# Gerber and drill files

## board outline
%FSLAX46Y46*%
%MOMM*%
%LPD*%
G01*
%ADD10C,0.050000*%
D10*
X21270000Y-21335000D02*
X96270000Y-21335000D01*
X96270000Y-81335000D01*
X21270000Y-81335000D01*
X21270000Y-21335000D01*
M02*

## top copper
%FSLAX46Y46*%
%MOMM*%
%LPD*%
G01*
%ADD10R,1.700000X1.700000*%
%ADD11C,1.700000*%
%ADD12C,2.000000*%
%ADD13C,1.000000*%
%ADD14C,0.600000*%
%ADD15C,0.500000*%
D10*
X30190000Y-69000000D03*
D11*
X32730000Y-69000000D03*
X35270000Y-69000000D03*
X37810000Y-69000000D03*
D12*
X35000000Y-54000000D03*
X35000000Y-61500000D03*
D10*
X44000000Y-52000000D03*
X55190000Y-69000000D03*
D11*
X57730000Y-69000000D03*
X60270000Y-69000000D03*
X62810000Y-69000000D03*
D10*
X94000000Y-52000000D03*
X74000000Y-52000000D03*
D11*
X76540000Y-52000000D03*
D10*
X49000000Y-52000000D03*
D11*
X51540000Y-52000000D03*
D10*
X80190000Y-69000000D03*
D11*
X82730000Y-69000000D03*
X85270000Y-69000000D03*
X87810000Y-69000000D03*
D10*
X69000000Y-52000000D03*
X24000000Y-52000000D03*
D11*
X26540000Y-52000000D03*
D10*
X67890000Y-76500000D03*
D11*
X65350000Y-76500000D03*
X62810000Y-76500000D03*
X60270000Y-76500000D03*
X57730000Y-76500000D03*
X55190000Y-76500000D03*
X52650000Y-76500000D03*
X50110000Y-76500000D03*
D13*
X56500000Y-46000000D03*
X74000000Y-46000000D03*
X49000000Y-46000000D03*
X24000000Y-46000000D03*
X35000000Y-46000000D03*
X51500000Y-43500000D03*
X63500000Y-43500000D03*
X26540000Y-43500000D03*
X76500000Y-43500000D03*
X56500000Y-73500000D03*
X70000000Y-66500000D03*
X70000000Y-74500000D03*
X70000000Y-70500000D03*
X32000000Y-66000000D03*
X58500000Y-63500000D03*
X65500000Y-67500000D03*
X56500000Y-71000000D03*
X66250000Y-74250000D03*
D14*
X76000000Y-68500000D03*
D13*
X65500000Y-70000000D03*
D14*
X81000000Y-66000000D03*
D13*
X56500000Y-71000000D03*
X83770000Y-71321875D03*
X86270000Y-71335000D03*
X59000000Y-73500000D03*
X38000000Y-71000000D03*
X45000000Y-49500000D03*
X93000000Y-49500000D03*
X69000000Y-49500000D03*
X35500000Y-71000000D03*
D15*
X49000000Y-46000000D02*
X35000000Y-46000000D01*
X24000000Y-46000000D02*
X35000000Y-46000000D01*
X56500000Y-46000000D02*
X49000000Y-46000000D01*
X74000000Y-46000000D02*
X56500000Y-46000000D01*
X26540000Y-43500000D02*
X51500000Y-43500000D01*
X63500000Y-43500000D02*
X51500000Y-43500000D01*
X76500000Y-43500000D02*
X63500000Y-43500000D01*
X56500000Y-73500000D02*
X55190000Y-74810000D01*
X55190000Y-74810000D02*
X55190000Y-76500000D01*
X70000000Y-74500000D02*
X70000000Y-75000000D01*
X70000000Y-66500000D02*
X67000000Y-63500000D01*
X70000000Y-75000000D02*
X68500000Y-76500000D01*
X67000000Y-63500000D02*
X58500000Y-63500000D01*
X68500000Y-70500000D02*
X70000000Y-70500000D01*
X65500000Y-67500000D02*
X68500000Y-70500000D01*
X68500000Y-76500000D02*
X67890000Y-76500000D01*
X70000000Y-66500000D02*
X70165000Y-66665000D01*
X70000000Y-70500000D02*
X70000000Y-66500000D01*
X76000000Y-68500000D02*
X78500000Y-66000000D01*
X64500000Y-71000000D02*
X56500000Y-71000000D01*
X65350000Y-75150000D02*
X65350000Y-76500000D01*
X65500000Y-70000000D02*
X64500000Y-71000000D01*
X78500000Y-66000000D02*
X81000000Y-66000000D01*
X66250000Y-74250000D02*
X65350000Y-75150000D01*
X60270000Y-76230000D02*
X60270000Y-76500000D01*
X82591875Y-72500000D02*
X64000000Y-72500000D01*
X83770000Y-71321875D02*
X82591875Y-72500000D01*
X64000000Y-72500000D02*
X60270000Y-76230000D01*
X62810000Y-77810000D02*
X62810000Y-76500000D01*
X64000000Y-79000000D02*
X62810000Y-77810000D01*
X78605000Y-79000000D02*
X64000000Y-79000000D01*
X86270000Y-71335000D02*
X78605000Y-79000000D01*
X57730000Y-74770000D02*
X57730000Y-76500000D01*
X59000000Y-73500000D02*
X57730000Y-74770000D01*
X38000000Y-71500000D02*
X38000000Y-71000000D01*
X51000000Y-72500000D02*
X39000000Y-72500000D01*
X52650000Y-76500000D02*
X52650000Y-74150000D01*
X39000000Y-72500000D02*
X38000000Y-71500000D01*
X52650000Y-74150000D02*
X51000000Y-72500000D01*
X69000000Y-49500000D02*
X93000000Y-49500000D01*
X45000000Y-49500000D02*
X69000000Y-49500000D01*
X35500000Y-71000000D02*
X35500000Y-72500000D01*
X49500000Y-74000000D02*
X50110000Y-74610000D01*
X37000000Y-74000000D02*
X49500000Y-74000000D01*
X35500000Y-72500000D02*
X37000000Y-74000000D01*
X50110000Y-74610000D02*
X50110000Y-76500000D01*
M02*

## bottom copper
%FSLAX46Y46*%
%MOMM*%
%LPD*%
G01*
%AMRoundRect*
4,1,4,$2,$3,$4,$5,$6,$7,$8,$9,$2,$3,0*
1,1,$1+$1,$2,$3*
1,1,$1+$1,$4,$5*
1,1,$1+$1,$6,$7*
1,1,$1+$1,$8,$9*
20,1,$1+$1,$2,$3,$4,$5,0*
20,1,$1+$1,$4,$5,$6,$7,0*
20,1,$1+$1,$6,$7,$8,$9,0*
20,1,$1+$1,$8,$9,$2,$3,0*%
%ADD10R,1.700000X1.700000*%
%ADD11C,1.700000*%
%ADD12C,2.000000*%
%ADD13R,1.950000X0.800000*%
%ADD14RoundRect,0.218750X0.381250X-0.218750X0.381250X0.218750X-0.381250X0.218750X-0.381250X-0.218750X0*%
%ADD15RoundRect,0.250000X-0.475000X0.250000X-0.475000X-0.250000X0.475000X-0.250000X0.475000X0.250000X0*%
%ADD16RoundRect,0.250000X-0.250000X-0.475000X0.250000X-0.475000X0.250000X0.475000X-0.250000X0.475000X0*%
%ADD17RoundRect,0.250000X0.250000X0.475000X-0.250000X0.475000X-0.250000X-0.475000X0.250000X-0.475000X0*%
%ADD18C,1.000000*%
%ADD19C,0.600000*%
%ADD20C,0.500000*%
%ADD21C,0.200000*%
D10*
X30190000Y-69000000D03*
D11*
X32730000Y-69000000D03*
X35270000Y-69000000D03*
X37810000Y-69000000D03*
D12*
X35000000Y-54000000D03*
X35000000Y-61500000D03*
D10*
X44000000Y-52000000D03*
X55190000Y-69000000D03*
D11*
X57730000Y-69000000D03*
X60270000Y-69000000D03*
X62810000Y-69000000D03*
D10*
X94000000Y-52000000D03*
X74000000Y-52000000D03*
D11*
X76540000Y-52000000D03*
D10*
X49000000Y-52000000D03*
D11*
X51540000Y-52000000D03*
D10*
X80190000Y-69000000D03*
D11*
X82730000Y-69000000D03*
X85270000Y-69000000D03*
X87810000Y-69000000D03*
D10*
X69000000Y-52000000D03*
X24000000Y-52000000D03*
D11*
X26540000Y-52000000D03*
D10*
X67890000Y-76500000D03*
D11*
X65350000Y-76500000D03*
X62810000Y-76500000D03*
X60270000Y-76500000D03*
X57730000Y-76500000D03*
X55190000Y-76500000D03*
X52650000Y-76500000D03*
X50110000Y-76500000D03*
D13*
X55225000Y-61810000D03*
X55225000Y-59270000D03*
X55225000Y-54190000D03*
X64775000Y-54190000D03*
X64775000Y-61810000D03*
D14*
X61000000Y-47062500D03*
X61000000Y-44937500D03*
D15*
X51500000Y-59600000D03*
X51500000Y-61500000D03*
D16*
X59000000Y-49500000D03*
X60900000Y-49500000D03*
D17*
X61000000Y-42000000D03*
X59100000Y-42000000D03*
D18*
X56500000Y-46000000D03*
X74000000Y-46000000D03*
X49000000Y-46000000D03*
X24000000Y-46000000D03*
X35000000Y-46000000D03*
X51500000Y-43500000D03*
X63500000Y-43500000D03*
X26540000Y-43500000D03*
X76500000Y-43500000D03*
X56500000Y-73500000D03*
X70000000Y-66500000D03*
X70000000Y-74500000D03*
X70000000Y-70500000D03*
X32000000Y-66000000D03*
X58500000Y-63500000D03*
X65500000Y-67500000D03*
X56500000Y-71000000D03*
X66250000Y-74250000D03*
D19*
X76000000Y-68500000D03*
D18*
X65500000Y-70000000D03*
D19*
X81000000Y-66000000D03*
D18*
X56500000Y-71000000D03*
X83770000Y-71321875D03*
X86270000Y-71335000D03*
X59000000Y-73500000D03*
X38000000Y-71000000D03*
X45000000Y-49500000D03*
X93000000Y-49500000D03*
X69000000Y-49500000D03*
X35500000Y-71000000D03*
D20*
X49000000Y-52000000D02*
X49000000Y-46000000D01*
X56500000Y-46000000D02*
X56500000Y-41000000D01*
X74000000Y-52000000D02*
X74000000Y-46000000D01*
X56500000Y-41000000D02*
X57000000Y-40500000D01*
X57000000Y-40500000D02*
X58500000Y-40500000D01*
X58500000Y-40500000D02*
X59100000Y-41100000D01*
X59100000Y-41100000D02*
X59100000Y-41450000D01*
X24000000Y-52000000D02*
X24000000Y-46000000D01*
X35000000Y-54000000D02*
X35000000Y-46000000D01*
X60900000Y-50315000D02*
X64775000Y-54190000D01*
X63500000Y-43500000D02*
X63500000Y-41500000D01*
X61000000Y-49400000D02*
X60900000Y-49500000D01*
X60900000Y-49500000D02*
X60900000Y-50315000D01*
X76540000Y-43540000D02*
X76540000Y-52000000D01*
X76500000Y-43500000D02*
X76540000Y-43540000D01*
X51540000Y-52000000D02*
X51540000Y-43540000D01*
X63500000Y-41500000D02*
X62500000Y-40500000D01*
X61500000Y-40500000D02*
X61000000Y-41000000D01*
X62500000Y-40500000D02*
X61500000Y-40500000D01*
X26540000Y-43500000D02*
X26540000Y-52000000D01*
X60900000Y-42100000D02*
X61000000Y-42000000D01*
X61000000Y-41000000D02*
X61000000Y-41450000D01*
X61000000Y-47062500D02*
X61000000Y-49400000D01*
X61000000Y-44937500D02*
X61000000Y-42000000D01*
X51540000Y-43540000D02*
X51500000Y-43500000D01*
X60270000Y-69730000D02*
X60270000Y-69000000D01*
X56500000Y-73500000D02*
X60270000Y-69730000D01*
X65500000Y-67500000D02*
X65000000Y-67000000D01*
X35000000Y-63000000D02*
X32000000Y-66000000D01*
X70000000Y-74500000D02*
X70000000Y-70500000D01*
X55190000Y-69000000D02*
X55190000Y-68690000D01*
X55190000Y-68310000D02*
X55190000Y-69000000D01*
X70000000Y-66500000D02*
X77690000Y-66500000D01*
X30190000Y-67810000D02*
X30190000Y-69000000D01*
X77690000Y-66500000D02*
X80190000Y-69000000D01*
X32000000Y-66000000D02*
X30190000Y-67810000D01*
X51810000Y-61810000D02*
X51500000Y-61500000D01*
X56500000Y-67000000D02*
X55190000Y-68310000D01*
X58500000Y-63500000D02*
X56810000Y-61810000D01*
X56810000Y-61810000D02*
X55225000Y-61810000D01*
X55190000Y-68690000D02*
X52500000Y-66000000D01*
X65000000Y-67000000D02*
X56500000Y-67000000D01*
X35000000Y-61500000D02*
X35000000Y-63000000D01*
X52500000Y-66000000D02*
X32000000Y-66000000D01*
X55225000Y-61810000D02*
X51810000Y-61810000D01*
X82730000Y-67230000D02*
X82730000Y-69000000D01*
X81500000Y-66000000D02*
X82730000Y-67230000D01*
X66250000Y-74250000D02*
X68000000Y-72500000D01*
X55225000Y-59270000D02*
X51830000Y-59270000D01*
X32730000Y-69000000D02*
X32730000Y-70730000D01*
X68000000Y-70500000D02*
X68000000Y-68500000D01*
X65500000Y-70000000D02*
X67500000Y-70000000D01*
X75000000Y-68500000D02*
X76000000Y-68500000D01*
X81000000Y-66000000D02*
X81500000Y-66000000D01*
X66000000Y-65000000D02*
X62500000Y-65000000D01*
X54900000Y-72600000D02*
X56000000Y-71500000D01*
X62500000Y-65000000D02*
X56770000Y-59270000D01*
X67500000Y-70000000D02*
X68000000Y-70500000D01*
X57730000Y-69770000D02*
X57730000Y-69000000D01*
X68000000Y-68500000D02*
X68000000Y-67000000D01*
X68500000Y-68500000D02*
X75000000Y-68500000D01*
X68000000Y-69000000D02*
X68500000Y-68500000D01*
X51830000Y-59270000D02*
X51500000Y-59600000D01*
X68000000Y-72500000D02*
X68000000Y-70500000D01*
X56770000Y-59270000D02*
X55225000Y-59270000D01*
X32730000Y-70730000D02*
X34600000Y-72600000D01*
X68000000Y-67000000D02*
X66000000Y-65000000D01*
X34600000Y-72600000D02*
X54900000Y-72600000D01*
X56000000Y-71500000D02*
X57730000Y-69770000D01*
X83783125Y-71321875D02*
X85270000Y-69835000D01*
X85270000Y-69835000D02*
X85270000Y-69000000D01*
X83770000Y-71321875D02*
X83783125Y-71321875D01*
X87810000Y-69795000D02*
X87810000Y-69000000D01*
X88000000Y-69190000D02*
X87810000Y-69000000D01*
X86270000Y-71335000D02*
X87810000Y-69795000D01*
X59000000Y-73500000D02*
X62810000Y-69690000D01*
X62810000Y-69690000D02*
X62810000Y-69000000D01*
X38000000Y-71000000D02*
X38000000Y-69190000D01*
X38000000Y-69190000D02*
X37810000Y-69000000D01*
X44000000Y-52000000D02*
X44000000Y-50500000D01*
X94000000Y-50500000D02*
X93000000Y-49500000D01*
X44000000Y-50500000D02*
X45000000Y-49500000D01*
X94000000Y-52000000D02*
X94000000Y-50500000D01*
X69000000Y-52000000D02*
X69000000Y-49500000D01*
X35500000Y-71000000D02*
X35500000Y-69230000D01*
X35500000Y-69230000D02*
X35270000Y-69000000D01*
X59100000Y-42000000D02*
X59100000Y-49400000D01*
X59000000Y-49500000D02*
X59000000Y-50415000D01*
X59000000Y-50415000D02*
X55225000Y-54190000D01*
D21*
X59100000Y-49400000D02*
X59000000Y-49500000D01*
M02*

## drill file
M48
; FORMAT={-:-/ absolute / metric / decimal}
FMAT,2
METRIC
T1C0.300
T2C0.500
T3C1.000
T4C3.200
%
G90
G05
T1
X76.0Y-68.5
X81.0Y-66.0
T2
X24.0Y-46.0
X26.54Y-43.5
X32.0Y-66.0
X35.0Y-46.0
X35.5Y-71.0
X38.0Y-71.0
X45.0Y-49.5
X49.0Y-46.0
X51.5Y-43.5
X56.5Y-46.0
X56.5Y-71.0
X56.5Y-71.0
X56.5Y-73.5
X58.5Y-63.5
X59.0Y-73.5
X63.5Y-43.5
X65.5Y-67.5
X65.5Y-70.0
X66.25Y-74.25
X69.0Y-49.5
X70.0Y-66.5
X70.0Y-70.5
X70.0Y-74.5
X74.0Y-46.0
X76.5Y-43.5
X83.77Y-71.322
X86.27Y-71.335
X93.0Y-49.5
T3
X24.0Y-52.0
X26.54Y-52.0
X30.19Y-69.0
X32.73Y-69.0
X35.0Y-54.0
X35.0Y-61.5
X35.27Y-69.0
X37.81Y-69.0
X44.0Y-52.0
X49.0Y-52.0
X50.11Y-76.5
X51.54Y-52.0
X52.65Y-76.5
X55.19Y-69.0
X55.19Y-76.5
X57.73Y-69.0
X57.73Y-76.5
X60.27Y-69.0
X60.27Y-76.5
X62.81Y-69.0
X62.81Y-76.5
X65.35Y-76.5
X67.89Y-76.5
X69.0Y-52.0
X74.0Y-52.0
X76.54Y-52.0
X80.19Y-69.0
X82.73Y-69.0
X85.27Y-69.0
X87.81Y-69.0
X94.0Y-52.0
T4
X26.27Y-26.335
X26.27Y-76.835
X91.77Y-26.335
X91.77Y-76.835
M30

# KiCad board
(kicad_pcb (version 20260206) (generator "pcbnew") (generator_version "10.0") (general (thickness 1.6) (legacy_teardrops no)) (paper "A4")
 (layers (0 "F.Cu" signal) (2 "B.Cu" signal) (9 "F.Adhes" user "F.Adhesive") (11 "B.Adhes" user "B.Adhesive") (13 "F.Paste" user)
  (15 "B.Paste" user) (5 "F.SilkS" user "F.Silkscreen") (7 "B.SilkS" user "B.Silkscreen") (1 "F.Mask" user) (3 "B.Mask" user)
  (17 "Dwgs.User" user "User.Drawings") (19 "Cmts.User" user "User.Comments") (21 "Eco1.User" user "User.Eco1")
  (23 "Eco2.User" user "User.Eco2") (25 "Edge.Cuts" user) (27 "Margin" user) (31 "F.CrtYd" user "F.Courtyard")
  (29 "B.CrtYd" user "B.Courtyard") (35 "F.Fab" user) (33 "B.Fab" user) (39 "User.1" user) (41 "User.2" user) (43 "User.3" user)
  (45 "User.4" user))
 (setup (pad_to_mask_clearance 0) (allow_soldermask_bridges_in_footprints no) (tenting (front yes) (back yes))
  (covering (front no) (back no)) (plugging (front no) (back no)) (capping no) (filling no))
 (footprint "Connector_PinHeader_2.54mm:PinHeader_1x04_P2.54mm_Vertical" (layer "F.Cu") (at 30.19 69 90)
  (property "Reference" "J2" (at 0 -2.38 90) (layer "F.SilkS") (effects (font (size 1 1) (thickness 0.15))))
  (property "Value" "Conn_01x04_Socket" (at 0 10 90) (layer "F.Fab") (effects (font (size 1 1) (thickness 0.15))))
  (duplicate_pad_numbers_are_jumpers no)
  (pad "1" thru_hole rect (at 0 0 90) (size 1.7 1.7) (drill 1) (layers "*.Cu" "*.Mask") (remove_unused_layers no) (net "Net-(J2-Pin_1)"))
  (pad "2" thru_hole circle (at 0 2.54 90) (size 1.7 1.7) (drill 1) (layers "*.Cu" "*.Mask") (remove_unused_layers no)
   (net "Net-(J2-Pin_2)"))
  (pad "3" thru_hole circle (at 0 5.08 90) (size 1.7 1.7) (drill 1) (layers "*.Cu" "*.Mask") (remove_unused_layers no)
   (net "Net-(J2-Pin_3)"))
  (pad "4" thru_hole circle (at 0 7.62 90) (size 1.7 1.7) (drill 1) (layers "*.Cu" "*.Mask") (remove_unused_layers no)
   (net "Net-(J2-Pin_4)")))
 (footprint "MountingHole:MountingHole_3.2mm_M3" (layer "F.Cu") (at 26.27 26.335)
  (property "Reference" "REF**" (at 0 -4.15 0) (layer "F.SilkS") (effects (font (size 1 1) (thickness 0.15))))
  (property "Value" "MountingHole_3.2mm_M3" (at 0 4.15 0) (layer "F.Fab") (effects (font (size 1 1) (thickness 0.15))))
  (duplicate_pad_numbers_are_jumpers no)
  (pad "" np_thru_hole circle (at 0 0) (size 3.2 3.2) (drill 3.2) (layers "*.Cu" "*.Mask")))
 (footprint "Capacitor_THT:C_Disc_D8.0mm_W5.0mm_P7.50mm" (layer "F.Cu") (at 35 54 -90)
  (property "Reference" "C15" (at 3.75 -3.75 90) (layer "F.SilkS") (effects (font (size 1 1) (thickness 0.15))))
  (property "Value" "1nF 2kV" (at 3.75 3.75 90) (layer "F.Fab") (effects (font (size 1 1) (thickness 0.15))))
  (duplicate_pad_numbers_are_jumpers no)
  (pad "1" thru_hole circle (at 0 0 270) (size 2 2) (drill 1) (layers "*.Cu" "*.Mask") (remove_unused_layers no) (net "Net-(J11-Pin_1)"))
  (pad "2" thru_hole circle (at 7.5 0 270) (size 2 2) (drill 1) (layers "*.Cu" "*.Mask") (remove_unused_layers no) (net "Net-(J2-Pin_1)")))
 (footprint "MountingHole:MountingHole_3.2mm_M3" (layer "F.Cu") (at 91.77 76.835)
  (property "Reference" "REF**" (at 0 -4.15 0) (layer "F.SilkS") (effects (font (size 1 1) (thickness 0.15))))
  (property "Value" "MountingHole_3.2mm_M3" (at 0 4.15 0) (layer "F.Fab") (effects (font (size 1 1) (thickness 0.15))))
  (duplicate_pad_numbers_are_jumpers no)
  (pad "" np_thru_hole circle (at 0 0) (size 3.2 3.2) (drill 3.2) (layers "*.Cu" "*.Mask")))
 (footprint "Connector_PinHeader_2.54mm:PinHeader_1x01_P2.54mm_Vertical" (layer "F.Cu") (at 44 52 90)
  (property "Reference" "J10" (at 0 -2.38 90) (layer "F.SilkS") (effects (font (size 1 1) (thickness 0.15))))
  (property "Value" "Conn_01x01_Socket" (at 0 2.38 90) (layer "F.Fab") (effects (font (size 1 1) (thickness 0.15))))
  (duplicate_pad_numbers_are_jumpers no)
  (pad "1" thru_hole rect (at 0 0 90) (size 1.7 1.7) (drill 1) (layers "*.Cu" "*.Mask") (remove_unused_layers no) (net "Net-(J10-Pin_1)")))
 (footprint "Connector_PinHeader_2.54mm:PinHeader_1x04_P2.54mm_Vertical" (layer "F.Cu") (at 55.19 69 90)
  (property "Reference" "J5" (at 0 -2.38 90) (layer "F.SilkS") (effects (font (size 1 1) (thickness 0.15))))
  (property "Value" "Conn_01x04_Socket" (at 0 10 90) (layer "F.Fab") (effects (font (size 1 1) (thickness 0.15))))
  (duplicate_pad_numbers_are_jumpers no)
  (pad "1" thru_hole rect (at 0 0 90) (size 1.7 1.7) (drill 1) (layers "*.Cu" "*.Mask") (remove_unused_layers no) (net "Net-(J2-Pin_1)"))
  (pad "2" thru_hole circle (at 0 2.54 90) (size 1.7 1.7) (drill 1) (layers "*.Cu" "*.Mask") (remove_unused_layers no)
   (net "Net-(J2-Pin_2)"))
  (pad "3" thru_hole circle (at 0 5.08 90) (size 1.7 1.7) (drill 1) (layers "*.Cu" "*.Mask") (remove_unused_layers no)
   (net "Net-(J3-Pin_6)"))
  (pad "4" thru_hole circle (at 0 7.62 90) (size 1.7 1.7) (drill 1) (layers "*.Cu" "*.Mask") (remove_unused_layers no)
   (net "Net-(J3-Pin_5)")))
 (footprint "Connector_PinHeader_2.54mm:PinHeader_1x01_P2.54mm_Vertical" (layer "F.Cu") (at 94 52 90)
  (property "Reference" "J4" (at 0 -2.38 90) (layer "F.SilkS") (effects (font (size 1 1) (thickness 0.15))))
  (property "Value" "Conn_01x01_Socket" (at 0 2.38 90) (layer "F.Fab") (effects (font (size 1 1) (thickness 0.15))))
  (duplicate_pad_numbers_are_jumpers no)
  (pad "1" thru_hole rect (at 0 0 90) (size 1.7 1.7) (drill 1) (layers "*.Cu" "*.Mask") (remove_unused_layers no) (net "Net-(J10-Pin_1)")))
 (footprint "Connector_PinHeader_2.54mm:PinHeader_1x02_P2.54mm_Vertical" (layer "F.Cu") (at 74 52 90)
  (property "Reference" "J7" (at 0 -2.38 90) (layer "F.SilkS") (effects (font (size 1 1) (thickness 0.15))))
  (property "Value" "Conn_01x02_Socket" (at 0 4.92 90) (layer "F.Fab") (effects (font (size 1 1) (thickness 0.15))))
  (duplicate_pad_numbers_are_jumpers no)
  (pad "1" thru_hole rect (at 0 0 90) (size 1.7 1.7) (drill 1) (layers "*.Cu" "*.Mask") (remove_unused_layers no) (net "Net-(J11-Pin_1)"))
  (pad "2" thru_hole circle (at 0 2.54 90) (size 1.7 1.7) (drill 1) (layers "*.Cu" "*.Mask") (remove_unused_layers no)
   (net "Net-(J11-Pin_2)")))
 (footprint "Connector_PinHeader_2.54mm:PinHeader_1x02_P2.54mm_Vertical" (layer "F.Cu") (at 49 52 90)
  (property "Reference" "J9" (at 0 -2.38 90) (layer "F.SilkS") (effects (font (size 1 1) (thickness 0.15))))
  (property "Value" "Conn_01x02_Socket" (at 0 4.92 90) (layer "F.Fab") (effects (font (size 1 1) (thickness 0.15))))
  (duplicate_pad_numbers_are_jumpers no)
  (pad "1" thru_hole rect (at 0 0 90) (size 1.7 1.7) (drill 1) (layers "*.Cu" "*.Mask") (remove_unused_layers no) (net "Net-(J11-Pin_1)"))
  (pad "2" thru_hole circle (at 0 2.54 90) (size 1.7 1.7) (drill 1) (layers "*.Cu" "*.Mask") (remove_unused_layers no)
   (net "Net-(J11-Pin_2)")))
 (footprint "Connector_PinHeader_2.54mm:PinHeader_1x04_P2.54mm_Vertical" (layer "F.Cu") (at 80.19 69 90)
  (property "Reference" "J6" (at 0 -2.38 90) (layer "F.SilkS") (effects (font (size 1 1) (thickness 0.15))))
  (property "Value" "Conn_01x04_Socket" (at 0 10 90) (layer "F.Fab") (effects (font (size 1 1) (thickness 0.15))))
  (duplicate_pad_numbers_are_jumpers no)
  (pad "1" thru_hole rect (at 0 0 90) (size 1.7 1.7) (drill 1) (layers "*.Cu" "*.Mask") (remove_unused_layers no) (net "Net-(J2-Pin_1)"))
  (pad "2" thru_hole circle (at 0 2.54 90) (size 1.7 1.7) (drill 1) (layers "*.Cu" "*.Mask") (remove_unused_layers no)
   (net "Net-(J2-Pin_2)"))
  (pad "3" thru_hole circle (at 0 5.08 90) (size 1.7 1.7) (drill 1) (layers "*.Cu" "*.Mask") (remove_unused_layers no)
   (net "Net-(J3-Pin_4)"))
  (pad "4" thru_hole circle (at 0 7.62 90) (size 1.7 1.7) (drill 1) (layers "*.Cu" "*.Mask") (remove_unused_layers no)
   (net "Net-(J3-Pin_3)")))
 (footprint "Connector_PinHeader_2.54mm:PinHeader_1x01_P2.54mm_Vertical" (layer "F.Cu") (at 69 52 90)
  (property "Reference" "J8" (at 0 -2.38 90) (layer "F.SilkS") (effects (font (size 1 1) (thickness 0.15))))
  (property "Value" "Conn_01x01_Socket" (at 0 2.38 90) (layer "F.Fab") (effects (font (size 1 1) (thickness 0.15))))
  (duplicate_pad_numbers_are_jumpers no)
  (pad "1" thru_hole rect (at 0 0 90) (size 1.7 1.7) (drill 1) (layers "*.Cu" "*.Mask") (remove_unused_layers no) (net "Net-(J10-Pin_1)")))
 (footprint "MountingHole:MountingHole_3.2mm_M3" (layer "F.Cu") (at 91.77 26.335)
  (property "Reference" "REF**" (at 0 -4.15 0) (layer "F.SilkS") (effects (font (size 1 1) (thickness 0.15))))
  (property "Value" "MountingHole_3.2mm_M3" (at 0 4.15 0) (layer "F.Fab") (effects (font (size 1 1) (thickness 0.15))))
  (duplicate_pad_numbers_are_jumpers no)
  (pad "" np_thru_hole circle (at 0 0) (size 3.2 3.2) (drill 3.2) (layers "*.Cu" "*.Mask")))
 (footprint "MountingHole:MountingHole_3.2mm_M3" (layer "F.Cu") (at 26.27 76.835)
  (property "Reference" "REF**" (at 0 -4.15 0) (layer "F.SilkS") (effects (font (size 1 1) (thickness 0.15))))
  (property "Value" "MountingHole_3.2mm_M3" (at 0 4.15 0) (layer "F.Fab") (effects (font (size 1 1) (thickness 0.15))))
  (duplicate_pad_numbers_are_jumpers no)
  (pad "" np_thru_hole circle (at 0 0) (size 3.2 3.2) (drill 3.2) (layers "*.Cu" "*.Mask")))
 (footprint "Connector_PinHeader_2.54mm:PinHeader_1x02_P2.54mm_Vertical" (layer "F.Cu") (at 24 52 90)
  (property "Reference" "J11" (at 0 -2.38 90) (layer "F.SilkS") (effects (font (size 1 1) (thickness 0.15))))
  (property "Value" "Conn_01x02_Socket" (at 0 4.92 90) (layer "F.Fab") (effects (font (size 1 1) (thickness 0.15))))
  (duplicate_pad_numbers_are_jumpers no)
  (pad "1" thru_hole rect (at 0 0 90) (size 1.7 1.7) (drill 1) (layers "*.Cu" "*.Mask") (remove_unused_layers no) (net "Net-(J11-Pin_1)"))
  (pad "2" thru_hole circle (at 0 2.54 90) (size 1.7 1.7) (drill 1) (layers "*.Cu" "*.Mask") (remove_unused_layers no)
   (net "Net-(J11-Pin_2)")))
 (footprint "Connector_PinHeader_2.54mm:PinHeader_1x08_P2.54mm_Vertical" (layer "F.Cu") (at 67.89 76.5 -90)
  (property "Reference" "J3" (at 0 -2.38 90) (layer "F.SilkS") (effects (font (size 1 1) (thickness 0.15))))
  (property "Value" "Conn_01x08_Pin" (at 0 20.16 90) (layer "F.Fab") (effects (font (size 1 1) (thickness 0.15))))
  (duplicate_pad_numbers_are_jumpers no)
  (pad "1" thru_hole rect (at 0 0 270) (size 1.7 1.7) (drill 1) (layers "*.Cu" "*.Mask") (remove_unused_layers no) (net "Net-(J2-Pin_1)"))
  (pad "2" thru_hole circle (at 0 2.54 270) (size 1.7 1.7) (drill 1) (layers "*.Cu" "*.Mask") (remove_unused_layers no)
   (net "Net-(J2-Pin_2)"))
  (pad "3" thru_hole circle (at 0 5.08 270) (size 1.7 1.7) (drill 1) (layers "*.Cu" "*.Mask") (remove_unused_layers no)
   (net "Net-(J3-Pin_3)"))
  (pad "4" thru_hole circle (at 0 7.62 270) (size 1.7 1.7) (drill 1) (layers "*.Cu" "*.Mask") (remove_unused_layers no)
   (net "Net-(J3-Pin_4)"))
  (pad "5" thru_hole circle (at 0 10.16 270) (size 1.7 1.7) (drill 1) (layers "*.Cu" "*.Mask") (remove_unused_layers no)
   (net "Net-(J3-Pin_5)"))
  (pad "6" thru_hole circle (at 0 12.7 270) (size 1.7 1.7) (drill 1) (layers "*.Cu" "*.Mask") (remove_unused_layers no)
   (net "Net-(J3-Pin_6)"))
  (pad "7" thru_hole circle (at 0 15.24 270) (size 1.7 1.7) (drill 1) (layers "*.Cu" "*.Mask") (remove_unused_layers no)
   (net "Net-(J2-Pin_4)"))
  (pad "8" thru_hole circle (at 0 17.78 270) (size 1.7 1.7) (drill 1) (layers "*.Cu" "*.Mask") (remove_unused_layers no)
   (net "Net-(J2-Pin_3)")))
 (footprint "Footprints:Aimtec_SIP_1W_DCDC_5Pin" (layer "B.Cu") (at 60 58 90)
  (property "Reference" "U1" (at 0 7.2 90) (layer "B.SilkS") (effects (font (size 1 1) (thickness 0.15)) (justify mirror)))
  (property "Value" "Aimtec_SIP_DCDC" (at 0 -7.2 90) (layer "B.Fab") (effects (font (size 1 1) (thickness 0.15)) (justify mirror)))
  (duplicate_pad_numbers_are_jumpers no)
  (pad "1" smd rect (at -3.81 -4.775 90) (size 0.8 1.95) (layers "B.Cu" "B.Mask" "B.Paste") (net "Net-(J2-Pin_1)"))
  (pad "2" smd rect (at -1.27 -4.775 90) (size 0.8 1.95) (layers "B.Cu" "B.Mask" "B.Paste") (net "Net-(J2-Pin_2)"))
  (pad "4" smd rect (at 3.81 -4.775 90) (size 0.8 1.95) (layers "B.Cu" "B.Mask" "B.Paste") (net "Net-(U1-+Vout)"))
  (pad "5" smd rect (at 3.81 4.775 90) (size 0.8 1.95) (layers "B.Cu" "B.Mask" "B.Paste") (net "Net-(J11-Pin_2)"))
  (pad "8" smd rect (at -3.81 4.775 90) (size 0.8 1.95) (layers "B.Cu" "B.Mask" "B.Paste") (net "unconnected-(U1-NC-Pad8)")))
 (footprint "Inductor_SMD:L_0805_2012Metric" (layer "B.Cu") (at 61 46 90)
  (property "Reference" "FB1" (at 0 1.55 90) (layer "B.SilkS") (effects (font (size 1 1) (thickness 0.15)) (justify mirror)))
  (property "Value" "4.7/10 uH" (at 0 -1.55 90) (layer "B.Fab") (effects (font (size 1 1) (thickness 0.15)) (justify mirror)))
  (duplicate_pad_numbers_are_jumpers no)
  (pad "1" smd roundrect (at -1.0625 0 90) (size 0.875 1.2) (layers "B.Cu" "B.Mask" "B.Paste") (roundrect_rratio 0.25)
   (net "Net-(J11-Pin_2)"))
  (pad "2" smd roundrect (at 1.0625 0 90) (size 0.875 1.2) (layers "B.Cu" "B.Mask" "B.Paste") (roundrect_rratio 0.25)
   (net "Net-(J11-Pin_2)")))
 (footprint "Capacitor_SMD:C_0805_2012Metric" (layer "B.Cu") (at 51.5 60.55 -90)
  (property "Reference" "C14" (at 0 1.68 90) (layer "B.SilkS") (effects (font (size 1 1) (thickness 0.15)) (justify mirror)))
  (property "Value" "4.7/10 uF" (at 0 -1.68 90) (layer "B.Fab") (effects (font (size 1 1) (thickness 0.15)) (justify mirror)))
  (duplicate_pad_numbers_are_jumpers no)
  (pad "1" smd roundrect (at -0.95 0 270) (size 1 1.45) (layers "B.Cu" "B.Mask" "B.Paste") (roundrect_rratio 0.25) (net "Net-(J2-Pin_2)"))
  (pad "2" smd roundrect (at 0.95 0 270) (size 1 1.45) (layers "B.Cu" "B.Mask" "B.Paste") (roundrect_rratio 0.25) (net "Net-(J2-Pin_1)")))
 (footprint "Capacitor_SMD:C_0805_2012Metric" (layer "B.Cu") (at 59.95 49.5)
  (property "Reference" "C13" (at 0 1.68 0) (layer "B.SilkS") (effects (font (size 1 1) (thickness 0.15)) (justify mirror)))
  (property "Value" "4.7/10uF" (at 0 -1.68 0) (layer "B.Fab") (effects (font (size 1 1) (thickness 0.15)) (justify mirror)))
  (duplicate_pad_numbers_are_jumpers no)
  (pad "1" smd roundrect (at -0.95 0) (size 1 1.45) (layers "B.Cu" "B.Mask" "B.Paste") (roundrect_rratio 0.25) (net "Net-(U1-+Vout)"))
  (pad "2" smd roundrect (at 0.95 0) (size 1 1.45) (layers "B.Cu" "B.Mask" "B.Paste") (roundrect_rratio 0.25) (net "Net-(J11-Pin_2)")))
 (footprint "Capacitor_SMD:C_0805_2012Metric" (layer "B.Cu") (at 60.05 42 180)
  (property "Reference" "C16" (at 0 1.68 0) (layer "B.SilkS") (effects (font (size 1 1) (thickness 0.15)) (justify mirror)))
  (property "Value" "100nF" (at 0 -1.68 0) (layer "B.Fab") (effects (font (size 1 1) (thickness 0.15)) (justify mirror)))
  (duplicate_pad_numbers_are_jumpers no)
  (pad "1" smd roundrect (at -0.95 0 180) (size 1 1.45) (layers "B.Cu" "B.Mask" "B.Paste") (roundrect_rratio 0.25) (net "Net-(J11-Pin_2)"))
  (pad "2" smd roundrect (at 0.95 0 180) (size 1 1.45) (layers "B.Cu" "B.Mask" "B.Paste") (roundrect_rratio 0.25) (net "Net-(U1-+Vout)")))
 (gr_rect (start 21.27 21.335) (end 96.27 81.335) (stroke (width 0.05) (type default)) (fill no) (layer "Edge.Cuts"))
 (segment (start 49 46) (end 35 46) (width 0.5) (layer "F.Cu") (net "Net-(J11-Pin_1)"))
 (segment (start 24 46) (end 35 46) (width 0.5) (layer "F.Cu") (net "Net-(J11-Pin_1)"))
 (segment (start 56.5 46) (end 49 46) (width 0.5) (layer "F.Cu") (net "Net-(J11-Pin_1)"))
 (segment (start 74 46) (end 56.5 46) (width 0.5) (layer "F.Cu") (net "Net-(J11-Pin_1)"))
 (via (at 56.5 46) (size 1) (drill 0.5) (layers "F.Cu" "B.Cu") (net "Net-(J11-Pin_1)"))
 (via (at 74 46) (size 1) (drill 0.5) (layers "F.Cu" "B.Cu") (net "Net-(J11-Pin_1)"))
 (via (at 49 46) (size 1) (drill 0.5) (layers "F.Cu" "B.Cu") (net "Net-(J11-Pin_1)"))
 (via (at 24 46) (size 1) (drill 0.5) (layers "F.Cu" "B.Cu") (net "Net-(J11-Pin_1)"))
 (via (at 35 46) (size 1) (drill 0.5) (layers "F.Cu" "B.Cu") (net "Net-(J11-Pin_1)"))
 (segment (start 49 52) (end 49 46) (width 0.5) (layer "B.Cu") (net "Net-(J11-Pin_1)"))
 (segment (start 56.5 46) (end 56.5 41) (width 0.5) (layer "B.Cu") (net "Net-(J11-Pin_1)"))
 (segment (start 74 52) (end 74 46) (width 0.5) (layer "B.Cu") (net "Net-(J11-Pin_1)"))
 (segment (start 56.5 41) (end 57 40.5) (width 0.5) (layer "B.Cu") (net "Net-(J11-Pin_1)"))
 (segment (start 57 40.5) (end 58.5 40.5) (width 0.5) (layer "B.Cu") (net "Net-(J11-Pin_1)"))
 (segment (start 58.5 40.5) (end 59.1 41.1) (width 0.5) (layer "B.Cu") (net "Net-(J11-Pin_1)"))
 (segment (start 59.1 41.1) (end 59.1 41.45) (width 0.5) (layer "B.Cu") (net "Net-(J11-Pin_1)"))
 (segment (start 24 52) (end 24 46) (width 0.5) (layer "B.Cu") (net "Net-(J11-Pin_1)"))
 (segment (start 35 54) (end 35 46) (width 0.5) (layer "B.Cu") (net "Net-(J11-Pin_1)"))
 (segment (start 26.54 43.5) (end 51.5 43.5) (width 0.5) (layer "F.Cu") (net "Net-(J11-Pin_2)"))
 (segment (start 63.5 43.5) (end 51.5 43.5) (width 0.5) (layer "F.Cu") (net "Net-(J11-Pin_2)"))
 (segment (start 76.5 43.5) (end 63.5 43.5) (width 0.5) (layer "F.Cu") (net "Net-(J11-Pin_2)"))
 (via (at 51.5 43.5) (size 1) (drill 0.5) (layers "F.Cu" "B.Cu") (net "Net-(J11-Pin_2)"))
 (via (at 63.5 43.5) (size 1) (drill 0.5) (layers "F.Cu" "B.Cu") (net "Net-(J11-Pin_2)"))
 (via (at 26.54 43.5) (size 1) (drill 0.5) (layers "F.Cu" "B.Cu") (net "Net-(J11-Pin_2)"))
 (via (at 76.5 43.5) (size 1) (drill 0.5) (layers "F.Cu" "B.Cu") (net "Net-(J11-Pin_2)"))
 (segment (start 60.9 50.315) (end 64.775 54.19) (width 0.5) (layer "B.Cu") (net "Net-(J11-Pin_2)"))
 (segment (start 63.5 43.5) (end 63.5 41.5) (width 0.5) (layer "B.Cu") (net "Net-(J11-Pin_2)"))
 (segment (start 61 49.4) (end 60.9 49.5) (width 0.5) (layer "B.Cu") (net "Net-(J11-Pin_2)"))
 (segment (start 60.9 49.5) (end 60.9 50.315) (width 0.5) (layer "B.Cu") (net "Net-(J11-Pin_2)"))
 (segment (start 76.54 43.54) (end 76.54 52) (width 0.5) (layer "B.Cu") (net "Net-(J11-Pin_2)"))
 (segment (start 76.5 43.5) (end 76.54 43.54) (width 0.5) (layer "B.Cu") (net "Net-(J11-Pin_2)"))
 (segment (start 51.54 52) (end 51.54 43.54) (width 0.5) (layer "B.Cu") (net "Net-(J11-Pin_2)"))
 (segment (start 63.5 41.5) (end 62.5 40.5) (width 0.5) (layer "B.Cu") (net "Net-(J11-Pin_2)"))
 (segment (start 61.5 40.5) (end 61 41) (width 0.5) (layer "B.Cu") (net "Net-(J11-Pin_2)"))
 (segment (start 62.5 40.5) (end 61.5 40.5) (width 0.5) (layer "B.Cu") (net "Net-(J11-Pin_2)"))
 (segment (start 26.54 43.5) (end 26.54 52) (width 0.5) (layer "B.Cu") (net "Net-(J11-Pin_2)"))
 (segment (start 60.9 42.1) (end 61 42) (width 0.5) (layer "B.Cu") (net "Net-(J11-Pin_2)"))
 (segment (start 61 41) (end 61 41.45) (width 0.5) (layer "B.Cu") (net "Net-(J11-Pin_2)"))
 (segment (start 61 47.0625) (end 61 49.4) (width 0.5) (layer "B.Cu") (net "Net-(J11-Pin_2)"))
 (segment (start 61 44.9375) (end 61 42) (width 0.5) (layer "B.Cu") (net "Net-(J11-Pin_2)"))
 (segment (start 51.54 43.54) (end 51.5 43.5) (width 0.5) (layer "B.Cu") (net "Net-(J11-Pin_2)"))
 (segment (start 56.5 73.5) (end 55.19 74.81) (width 0.5) (layer "F.Cu") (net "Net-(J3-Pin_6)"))
 (segment (start 55.19 74.81) (end 55.19 76.5) (width 0.5) (layer "F.Cu") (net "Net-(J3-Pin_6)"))
 (via (at 56.5 73.5) (size 1) (drill 0.5) (layers "F.Cu" "B.Cu") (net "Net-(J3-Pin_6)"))
 (segment (start 60.27 69.73) (end 60.27 69) (width 0.5) (layer "B.Cu") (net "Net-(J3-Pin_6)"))
 (segment (start 56.5 73.5) (end 60.27 69.73) (width 0.5) (layer "B.Cu") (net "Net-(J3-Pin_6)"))
 (segment (start 70 74.5) (end 70 75) (width 0.5) (layer "F.Cu") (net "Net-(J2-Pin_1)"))
 (segment (start 70 66.5) (end 67 63.5) (width 0.5) (layer "F.Cu") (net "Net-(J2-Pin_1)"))
 (segment (start 70 75) (end 68.5 76.5) (width 0.5) (layer "F.Cu") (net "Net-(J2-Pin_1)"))
 (segment (start 67 63.5) (end 58.5 63.5) (width 0.5) (layer "F.Cu") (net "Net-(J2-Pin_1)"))
 (segment (start 68.5 70.5) (end 70 70.5) (width 0.5) (layer "F.Cu") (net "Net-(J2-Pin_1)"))
 (segment (start 65.5 67.5) (end 68.5 70.5) (width 0.5) (layer "F.Cu") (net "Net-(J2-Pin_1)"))
 (segment (start 68.5 76.5) (end 67.89 76.5) (width 0.5) (layer "F.Cu") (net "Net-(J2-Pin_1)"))
 (segment (start 70 66.5) (end 70.165 66.665) (width 0.5) (layer "F.Cu") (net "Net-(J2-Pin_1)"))
 (segment (start 70 70.5) (end 70 66.5) (width 0.5) (layer "F.Cu") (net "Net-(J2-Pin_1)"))
 (via (at 70 66.5) (size 1) (drill 0.5) (layers "F.Cu" "B.Cu") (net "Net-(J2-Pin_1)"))
 (via (at 70 74.5) (size 1) (drill 0.5) (layers "F.Cu" "B.Cu") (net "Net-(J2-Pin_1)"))
 (via (at 70 70.5) (size 1) (drill 0.5) (layers "F.Cu" "B.Cu") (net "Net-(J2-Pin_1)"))
 (via (at 32 66) (size 1) (drill 0.5) (layers "F.Cu" "B.Cu") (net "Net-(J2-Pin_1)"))
 (via (at 58.5 63.5) (size 1) (drill 0.5) (layers "F.Cu" "B.Cu") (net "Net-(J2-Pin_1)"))
 (via (at 65.5 67.5) (size 1) (drill 0.5) (layers "F.Cu" "B.Cu") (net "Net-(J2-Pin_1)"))
 (segment (start 65.5 67.5) (end 65 67) (width 0.5) (layer "B.Cu") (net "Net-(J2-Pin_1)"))
 (segment (start 35 63) (end 32 66) (width 0.5) (layer "B.Cu") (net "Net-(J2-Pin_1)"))
 (segment (start 70 74.5) (end 70 70.5) (width 0.5) (layer "B.Cu") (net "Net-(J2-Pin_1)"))
 (segment (start 55.19 69) (end 55.19 68.69) (width 0.5) (layer "B.Cu") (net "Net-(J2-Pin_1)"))
 (segment (start 55.19 68.31) (end 55.19 69) (width 0.5) (layer "B.Cu") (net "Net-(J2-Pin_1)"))
 (segment (start 70 66.5) (end 77.69 66.5) (width 0.5) (layer "B.Cu") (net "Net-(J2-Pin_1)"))
 (segment (start 30.19 67.81) (end 30.19 69) (width 0.5) (layer "B.Cu") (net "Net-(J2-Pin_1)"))
 (segment (start 77.69 66.5) (end 80.19 69) (width 0.5) (layer "B.Cu") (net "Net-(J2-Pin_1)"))
 (segment (start 32 66) (end 30.19 67.81) (width 0.5) (layer "B.Cu") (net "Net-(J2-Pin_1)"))
 (segment (start 51.81 61.81) (end 51.5 61.5) (width 0.5) (layer "B.Cu") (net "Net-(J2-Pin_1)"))
 (segment (start 56.5 67) (end 55.19 68.31) (width 0.5) (layer "B.Cu") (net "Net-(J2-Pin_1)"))
 (segment (start 58.5 63.5) (end 56.81 61.81) (width 0.5) (layer "B.Cu") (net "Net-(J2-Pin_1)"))
 (segment (start 56.81 61.81) (end 55.225 61.81) (width 0.5) (layer "B.Cu") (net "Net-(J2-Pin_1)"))
 (segment (start 55.19 68.69) (end 52.5 66) (width 0.5) (layer "B.Cu") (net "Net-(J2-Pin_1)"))
 (segment (start 65 67) (end 56.5 67) (width 0.5) (layer "B.Cu") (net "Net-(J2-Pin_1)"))
 (segment (start 35 61.5) (end 35 63) (width 0.5) (layer "B.Cu") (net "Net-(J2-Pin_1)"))
 (segment (start 52.5 66) (end 32 66) (width 0.5) (layer "B.Cu") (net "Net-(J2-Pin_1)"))
 (segment (start 55.225 61.81) (end 51.81 61.81) (width 0.5) (layer "B.Cu") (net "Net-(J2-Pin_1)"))
 (segment (start 76 68.5) (end 78.5 66) (width 0.5) (layer "F.Cu") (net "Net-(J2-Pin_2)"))
 (segment (start 64.5 71) (end 56.5 71) (width 0.5) (layer "F.Cu") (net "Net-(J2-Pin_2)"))
 (segment (start 65.35 75.15) (end 65.35 76.5) (width 0.5) (layer "F.Cu") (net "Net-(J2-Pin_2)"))
 (segment (start 65.5 70) (end 64.5 71) (width 0.5) (layer "F.Cu") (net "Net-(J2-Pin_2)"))
 (segment (start 78.5 66) (end 81 66) (width 0.5) (layer "F.Cu") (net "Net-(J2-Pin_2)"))
 (segment (start 66.25 74.25) (end 65.35 75.15) (width 0.5) (layer "F.Cu") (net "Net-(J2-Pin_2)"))
 (via (at 56.5 71) (size 1) (drill 0.5) (layers "F.Cu" "B.Cu") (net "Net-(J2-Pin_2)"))
 (via (at 66.25 74.25) (size 1) (drill 0.5) (layers "F.Cu" "B.Cu") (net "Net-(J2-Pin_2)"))
 (via (at 76 68.5) (size 0.6) (drill 0.3) (layers "F.Cu" "B.Cu") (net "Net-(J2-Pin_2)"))
 (via (at 65.5 70) (size 1) (drill 0.5) (layers "F.Cu" "B.Cu") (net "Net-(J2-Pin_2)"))
 (via (at 81 66) (size 0.6) (drill 0.3) (layers "F.Cu" "B.Cu") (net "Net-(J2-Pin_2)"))
 (via (at 56.5 71) (size 1) (drill 0.5) (layers "F.Cu" "B.Cu") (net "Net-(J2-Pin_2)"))
 (segment (start 82.73 67.23) (end 82.73 69) (width 0.5) (layer "B.Cu") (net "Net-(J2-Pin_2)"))
 (segment (start 81.5 66) (end 82.73 67.23) (width 0.5) (layer "B.Cu") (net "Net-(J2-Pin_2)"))
 (segment (start 66.25 74.25) (end 68 72.5) (width 0.5) (layer "B.Cu") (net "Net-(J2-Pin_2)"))
 (segment (start 55.225 59.27) (end 51.83 59.27) (width 0.5) (layer "B.Cu") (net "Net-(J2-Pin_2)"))
 (segment (start 32.73 69) (end 32.73 70.73) (width 0.5) (layer "B.Cu") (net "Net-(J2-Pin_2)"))
 (segment (start 68 70.5) (end 68 68.5) (width 0.5) (layer "B.Cu") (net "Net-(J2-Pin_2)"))
 (segment (start 65.5 70) (end 67.5 70) (width 0.5) (layer "B.Cu") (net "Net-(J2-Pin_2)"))
 (segment (start 75 68.5) (end 76 68.5) (width 0.5) (layer "B.Cu") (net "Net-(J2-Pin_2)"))
 (segment (start 81 66) (end 81.5 66) (width 0.5) (layer "B.Cu") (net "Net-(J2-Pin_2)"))
 (segment (start 66 65) (end 62.5 65) (width 0.5) (layer "B.Cu") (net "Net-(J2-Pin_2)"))
 (segment (start 54.9 72.6) (end 56 71.5) (width 0.5) (layer "B.Cu") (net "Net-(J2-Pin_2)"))
 (segment (start 62.5 65) (end 56.77 59.27) (width 0.5) (layer "B.Cu") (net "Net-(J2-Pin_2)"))
 (segment (start 67.5 70) (end 68 70.5) (width 0.5) (layer "B.Cu") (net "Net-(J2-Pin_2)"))
 (segment (start 57.73 69.77) (end 57.73 69) (width 0.5) (layer "B.Cu") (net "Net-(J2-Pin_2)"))
 (segment (start 68 68.5) (end 68 67) (width 0.5) (layer "B.Cu") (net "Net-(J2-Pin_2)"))
 (segment (start 68.5 68.5) (end 75 68.5) (width 0.5) (layer "B.Cu") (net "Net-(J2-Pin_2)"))
 (segment (start 68 69) (end 68.5 68.5) (width 0.5) (layer "B.Cu") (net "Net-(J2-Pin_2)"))
 (segment (start 51.83 59.27) (end 51.5 59.6) (width 0.5) (layer "B.Cu") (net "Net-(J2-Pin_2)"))
 (segment (start 68 72.5) (end 68 70.5) (width 0.5) (layer "B.Cu") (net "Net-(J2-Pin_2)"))
 (segment (start 56.77 59.27) (end 55.225 59.27) (width 0.5) (layer "B.Cu") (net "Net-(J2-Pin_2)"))
 (segment (start 32.73 70.73) (end 34.6 72.6) (width 0.5) (layer "B.Cu") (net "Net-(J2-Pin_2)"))
 (segment (start 68 67) (end 66 65) (width 0.5) (layer "B.Cu") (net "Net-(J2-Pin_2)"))
 (segment (start 34.6 72.6) (end 54.9 72.6) (width 0.5) (layer "B.Cu") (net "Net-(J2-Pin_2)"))
 (segment (start 56 71.5) (end 57.73 69.77) (width 0.5) (layer "B.Cu") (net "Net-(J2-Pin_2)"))
 (segment (start 60.27 76.23) (end 60.27 76.5) (width 0.5) (layer "F.Cu") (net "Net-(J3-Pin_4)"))
 (segment (start 82.591875 72.5) (end 64 72.5) (width 0.5) (layer "F.Cu") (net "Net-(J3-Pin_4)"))
 (segment (start 83.77 71.321875) (end 82.591875 72.5) (width 0.5) (layer "F.Cu") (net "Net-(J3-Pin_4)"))
 (segment (start 64 72.5) (end 60.27 76.23) (width 0.5) (layer "F.Cu") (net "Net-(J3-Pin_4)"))
 (via (at 83.77 71.321875) (size 1) (drill 0.5) (layers "F.Cu" "B.Cu") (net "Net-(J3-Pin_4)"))
 (segment (start 83.783125 71.321875) (end 85.27 69.835) (width 0.5) (layer "B.Cu") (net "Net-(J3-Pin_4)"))
 (segment (start 85.27 69.835) (end 85.27 69) (width 0.5) (layer "B.Cu") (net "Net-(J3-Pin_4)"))
 (segment (start 83.77 71.321875) (end 83.783125 71.321875) (width 0.5) (layer "B.Cu") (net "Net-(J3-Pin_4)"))
 (segment (start 62.81 77.81) (end 62.81 76.5) (width 0.5) (layer "F.Cu") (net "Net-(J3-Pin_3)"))
 (segment (start 64 79) (end 62.81 77.81) (width 0.5) (layer "F.Cu") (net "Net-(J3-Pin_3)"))
 (segment (start 78.605 79) (end 64 79) (width 0.5) (layer "F.Cu") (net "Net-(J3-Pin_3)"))
 (segment (start 86.27 71.335) (end 78.605 79) (width 0.5) (layer "F.Cu") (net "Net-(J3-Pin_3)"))
 (via (at 86.27 71.335) (size 1) (drill 0.5) (layers "F.Cu" "B.Cu") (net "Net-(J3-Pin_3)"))
 (segment (start 87.81 69.795) (end 87.81 69) (width 0.5) (layer "B.Cu") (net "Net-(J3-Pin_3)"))
 (segment (start 88 69.19) (end 87.81 69) (width 0.5) (layer "B.Cu") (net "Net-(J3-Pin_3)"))
 (segment (start 86.27 71.335) (end 87.81 69.795) (width 0.5) (layer "B.Cu") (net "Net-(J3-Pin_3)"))
 (segment (start 57.73 74.77) (end 57.73 76.5) (width 0.5) (layer "F.Cu") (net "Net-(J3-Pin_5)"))
 (segment (start 59 73.5) (end 57.73 74.77) (width 0.5) (layer "F.Cu") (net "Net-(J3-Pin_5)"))
 (via (at 59 73.5) (size 1) (drill 0.5) (layers "F.Cu" "B.Cu") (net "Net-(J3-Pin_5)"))
 (segment (start 59 73.5) (end 62.81 69.69) (width 0.5) (layer "B.Cu") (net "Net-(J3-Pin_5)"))
 (segment (start 62.81 69.69) (end 62.81 69) (width 0.5) (layer "B.Cu") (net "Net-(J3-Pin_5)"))
 (segment (start 38 71.5) (end 38 71) (width 0.5) (layer "F.Cu") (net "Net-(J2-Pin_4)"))
 (segment (start 51 72.5) (end 39 72.5) (width 0.5) (layer "F.Cu") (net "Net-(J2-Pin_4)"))
 (segment (start 52.65 76.5) (end 52.65 74.15) (width 0.5) (layer "F.Cu") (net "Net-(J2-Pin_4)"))
 (segment (start 39 72.5) (end 38 71.5) (width 0.5) (layer "F.Cu") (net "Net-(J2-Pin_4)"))
 (segment (start 52.65 74.15) (end 51 72.5) (width 0.5) (layer "F.Cu") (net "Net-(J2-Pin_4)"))
 (via (at 38 71) (size 1) (drill 0.5) (layers "F.Cu" "B.Cu") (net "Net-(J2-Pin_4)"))
 (segment (start 38 71) (end 38 69.19) (width 0.5) (layer "B.Cu") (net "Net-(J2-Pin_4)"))
 (segment (start 38 69.19) (end 37.81 69) (width 0.5) (layer "B.Cu") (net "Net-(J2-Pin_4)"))
 (segment (start 69 49.5) (end 93 49.5) (width 0.5) (layer "F.Cu") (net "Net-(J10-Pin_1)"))
 (segment (start 45 49.5) (end 69 49.5) (width 0.5) (layer "F.Cu") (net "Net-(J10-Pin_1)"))
 (via (at 45 49.5) (size 1) (drill 0.5) (layers "F.Cu" "B.Cu") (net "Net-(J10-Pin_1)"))
 (via (at 93 49.5) (size 1) (drill 0.5) (layers "F.Cu" "B.Cu") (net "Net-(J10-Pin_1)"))
 (via (at 69 49.5) (size 1) (drill 0.5) (layers "F.Cu" "B.Cu") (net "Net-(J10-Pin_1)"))
 (segment (start 44 52) (end 44 50.5) (width 0.5) (layer "B.Cu") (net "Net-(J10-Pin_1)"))
 (segment (start 94 50.5) (end 93 49.5) (width 0.5) (layer "B.Cu") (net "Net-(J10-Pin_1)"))
 (segment (start 44 50.5) (end 45 49.5) (width 0.5) (layer "B.Cu") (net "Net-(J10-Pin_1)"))
 (segment (start 94 52) (end 94 50.5) (width 0.5) (layer "B.Cu") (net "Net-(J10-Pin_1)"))
 (segment (start 69 52) (end 69 49.5) (width 0.5) (layer "B.Cu") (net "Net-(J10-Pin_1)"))
 (segment (start 35.5 71) (end 35.5 72.5) (width 0.5) (layer "F.Cu") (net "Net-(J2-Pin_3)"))
 (segment (start 49.5 74) (end 50.11 74.61) (width 0.5) (layer "F.Cu") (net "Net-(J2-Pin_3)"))
 (segment (start 37 74) (end 49.5 74) (width 0.5) (layer "F.Cu") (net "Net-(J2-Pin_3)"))
 (segment (start 35.5 72.5) (end 37 74) (width 0.5) (layer "F.Cu") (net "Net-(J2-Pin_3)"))
 (segment (start 50.11 74.61) (end 50.11 76.5) (width 0.5) (layer "F.Cu") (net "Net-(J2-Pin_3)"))
 (via (at 35.5 71) (size 1) (drill 0.5) (layers "F.Cu" "B.Cu") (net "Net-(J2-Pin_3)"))
 (segment (start 35.5 71) (end 35.5 69.23) (width 0.5) (layer "B.Cu") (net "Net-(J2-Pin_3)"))
 (segment (start 35.5 69.23) (end 35.27 69) (width 0.5) (layer "B.Cu") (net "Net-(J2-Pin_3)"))
 (segment (start 59.1 42) (end 59.1 49.4) (width 0.5) (layer "B.Cu") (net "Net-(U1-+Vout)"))
 (segment (start 59 49.5) (end 59 50.415) (width 0.5) (layer "B.Cu") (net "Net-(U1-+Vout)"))
 (segment (start 59 50.415) (end 55.225 54.19) (width 0.5) (layer "B.Cu") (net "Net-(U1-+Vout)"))
 (segment (start 59.1 49.4) (end 59 49.5) (width 0.2) (layer "B.Cu") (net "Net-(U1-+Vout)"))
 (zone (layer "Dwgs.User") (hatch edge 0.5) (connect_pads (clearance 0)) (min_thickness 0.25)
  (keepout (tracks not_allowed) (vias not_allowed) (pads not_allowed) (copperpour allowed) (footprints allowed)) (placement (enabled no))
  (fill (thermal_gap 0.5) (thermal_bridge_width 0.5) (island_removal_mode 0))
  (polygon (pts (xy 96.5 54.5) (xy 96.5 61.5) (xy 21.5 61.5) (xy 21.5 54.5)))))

